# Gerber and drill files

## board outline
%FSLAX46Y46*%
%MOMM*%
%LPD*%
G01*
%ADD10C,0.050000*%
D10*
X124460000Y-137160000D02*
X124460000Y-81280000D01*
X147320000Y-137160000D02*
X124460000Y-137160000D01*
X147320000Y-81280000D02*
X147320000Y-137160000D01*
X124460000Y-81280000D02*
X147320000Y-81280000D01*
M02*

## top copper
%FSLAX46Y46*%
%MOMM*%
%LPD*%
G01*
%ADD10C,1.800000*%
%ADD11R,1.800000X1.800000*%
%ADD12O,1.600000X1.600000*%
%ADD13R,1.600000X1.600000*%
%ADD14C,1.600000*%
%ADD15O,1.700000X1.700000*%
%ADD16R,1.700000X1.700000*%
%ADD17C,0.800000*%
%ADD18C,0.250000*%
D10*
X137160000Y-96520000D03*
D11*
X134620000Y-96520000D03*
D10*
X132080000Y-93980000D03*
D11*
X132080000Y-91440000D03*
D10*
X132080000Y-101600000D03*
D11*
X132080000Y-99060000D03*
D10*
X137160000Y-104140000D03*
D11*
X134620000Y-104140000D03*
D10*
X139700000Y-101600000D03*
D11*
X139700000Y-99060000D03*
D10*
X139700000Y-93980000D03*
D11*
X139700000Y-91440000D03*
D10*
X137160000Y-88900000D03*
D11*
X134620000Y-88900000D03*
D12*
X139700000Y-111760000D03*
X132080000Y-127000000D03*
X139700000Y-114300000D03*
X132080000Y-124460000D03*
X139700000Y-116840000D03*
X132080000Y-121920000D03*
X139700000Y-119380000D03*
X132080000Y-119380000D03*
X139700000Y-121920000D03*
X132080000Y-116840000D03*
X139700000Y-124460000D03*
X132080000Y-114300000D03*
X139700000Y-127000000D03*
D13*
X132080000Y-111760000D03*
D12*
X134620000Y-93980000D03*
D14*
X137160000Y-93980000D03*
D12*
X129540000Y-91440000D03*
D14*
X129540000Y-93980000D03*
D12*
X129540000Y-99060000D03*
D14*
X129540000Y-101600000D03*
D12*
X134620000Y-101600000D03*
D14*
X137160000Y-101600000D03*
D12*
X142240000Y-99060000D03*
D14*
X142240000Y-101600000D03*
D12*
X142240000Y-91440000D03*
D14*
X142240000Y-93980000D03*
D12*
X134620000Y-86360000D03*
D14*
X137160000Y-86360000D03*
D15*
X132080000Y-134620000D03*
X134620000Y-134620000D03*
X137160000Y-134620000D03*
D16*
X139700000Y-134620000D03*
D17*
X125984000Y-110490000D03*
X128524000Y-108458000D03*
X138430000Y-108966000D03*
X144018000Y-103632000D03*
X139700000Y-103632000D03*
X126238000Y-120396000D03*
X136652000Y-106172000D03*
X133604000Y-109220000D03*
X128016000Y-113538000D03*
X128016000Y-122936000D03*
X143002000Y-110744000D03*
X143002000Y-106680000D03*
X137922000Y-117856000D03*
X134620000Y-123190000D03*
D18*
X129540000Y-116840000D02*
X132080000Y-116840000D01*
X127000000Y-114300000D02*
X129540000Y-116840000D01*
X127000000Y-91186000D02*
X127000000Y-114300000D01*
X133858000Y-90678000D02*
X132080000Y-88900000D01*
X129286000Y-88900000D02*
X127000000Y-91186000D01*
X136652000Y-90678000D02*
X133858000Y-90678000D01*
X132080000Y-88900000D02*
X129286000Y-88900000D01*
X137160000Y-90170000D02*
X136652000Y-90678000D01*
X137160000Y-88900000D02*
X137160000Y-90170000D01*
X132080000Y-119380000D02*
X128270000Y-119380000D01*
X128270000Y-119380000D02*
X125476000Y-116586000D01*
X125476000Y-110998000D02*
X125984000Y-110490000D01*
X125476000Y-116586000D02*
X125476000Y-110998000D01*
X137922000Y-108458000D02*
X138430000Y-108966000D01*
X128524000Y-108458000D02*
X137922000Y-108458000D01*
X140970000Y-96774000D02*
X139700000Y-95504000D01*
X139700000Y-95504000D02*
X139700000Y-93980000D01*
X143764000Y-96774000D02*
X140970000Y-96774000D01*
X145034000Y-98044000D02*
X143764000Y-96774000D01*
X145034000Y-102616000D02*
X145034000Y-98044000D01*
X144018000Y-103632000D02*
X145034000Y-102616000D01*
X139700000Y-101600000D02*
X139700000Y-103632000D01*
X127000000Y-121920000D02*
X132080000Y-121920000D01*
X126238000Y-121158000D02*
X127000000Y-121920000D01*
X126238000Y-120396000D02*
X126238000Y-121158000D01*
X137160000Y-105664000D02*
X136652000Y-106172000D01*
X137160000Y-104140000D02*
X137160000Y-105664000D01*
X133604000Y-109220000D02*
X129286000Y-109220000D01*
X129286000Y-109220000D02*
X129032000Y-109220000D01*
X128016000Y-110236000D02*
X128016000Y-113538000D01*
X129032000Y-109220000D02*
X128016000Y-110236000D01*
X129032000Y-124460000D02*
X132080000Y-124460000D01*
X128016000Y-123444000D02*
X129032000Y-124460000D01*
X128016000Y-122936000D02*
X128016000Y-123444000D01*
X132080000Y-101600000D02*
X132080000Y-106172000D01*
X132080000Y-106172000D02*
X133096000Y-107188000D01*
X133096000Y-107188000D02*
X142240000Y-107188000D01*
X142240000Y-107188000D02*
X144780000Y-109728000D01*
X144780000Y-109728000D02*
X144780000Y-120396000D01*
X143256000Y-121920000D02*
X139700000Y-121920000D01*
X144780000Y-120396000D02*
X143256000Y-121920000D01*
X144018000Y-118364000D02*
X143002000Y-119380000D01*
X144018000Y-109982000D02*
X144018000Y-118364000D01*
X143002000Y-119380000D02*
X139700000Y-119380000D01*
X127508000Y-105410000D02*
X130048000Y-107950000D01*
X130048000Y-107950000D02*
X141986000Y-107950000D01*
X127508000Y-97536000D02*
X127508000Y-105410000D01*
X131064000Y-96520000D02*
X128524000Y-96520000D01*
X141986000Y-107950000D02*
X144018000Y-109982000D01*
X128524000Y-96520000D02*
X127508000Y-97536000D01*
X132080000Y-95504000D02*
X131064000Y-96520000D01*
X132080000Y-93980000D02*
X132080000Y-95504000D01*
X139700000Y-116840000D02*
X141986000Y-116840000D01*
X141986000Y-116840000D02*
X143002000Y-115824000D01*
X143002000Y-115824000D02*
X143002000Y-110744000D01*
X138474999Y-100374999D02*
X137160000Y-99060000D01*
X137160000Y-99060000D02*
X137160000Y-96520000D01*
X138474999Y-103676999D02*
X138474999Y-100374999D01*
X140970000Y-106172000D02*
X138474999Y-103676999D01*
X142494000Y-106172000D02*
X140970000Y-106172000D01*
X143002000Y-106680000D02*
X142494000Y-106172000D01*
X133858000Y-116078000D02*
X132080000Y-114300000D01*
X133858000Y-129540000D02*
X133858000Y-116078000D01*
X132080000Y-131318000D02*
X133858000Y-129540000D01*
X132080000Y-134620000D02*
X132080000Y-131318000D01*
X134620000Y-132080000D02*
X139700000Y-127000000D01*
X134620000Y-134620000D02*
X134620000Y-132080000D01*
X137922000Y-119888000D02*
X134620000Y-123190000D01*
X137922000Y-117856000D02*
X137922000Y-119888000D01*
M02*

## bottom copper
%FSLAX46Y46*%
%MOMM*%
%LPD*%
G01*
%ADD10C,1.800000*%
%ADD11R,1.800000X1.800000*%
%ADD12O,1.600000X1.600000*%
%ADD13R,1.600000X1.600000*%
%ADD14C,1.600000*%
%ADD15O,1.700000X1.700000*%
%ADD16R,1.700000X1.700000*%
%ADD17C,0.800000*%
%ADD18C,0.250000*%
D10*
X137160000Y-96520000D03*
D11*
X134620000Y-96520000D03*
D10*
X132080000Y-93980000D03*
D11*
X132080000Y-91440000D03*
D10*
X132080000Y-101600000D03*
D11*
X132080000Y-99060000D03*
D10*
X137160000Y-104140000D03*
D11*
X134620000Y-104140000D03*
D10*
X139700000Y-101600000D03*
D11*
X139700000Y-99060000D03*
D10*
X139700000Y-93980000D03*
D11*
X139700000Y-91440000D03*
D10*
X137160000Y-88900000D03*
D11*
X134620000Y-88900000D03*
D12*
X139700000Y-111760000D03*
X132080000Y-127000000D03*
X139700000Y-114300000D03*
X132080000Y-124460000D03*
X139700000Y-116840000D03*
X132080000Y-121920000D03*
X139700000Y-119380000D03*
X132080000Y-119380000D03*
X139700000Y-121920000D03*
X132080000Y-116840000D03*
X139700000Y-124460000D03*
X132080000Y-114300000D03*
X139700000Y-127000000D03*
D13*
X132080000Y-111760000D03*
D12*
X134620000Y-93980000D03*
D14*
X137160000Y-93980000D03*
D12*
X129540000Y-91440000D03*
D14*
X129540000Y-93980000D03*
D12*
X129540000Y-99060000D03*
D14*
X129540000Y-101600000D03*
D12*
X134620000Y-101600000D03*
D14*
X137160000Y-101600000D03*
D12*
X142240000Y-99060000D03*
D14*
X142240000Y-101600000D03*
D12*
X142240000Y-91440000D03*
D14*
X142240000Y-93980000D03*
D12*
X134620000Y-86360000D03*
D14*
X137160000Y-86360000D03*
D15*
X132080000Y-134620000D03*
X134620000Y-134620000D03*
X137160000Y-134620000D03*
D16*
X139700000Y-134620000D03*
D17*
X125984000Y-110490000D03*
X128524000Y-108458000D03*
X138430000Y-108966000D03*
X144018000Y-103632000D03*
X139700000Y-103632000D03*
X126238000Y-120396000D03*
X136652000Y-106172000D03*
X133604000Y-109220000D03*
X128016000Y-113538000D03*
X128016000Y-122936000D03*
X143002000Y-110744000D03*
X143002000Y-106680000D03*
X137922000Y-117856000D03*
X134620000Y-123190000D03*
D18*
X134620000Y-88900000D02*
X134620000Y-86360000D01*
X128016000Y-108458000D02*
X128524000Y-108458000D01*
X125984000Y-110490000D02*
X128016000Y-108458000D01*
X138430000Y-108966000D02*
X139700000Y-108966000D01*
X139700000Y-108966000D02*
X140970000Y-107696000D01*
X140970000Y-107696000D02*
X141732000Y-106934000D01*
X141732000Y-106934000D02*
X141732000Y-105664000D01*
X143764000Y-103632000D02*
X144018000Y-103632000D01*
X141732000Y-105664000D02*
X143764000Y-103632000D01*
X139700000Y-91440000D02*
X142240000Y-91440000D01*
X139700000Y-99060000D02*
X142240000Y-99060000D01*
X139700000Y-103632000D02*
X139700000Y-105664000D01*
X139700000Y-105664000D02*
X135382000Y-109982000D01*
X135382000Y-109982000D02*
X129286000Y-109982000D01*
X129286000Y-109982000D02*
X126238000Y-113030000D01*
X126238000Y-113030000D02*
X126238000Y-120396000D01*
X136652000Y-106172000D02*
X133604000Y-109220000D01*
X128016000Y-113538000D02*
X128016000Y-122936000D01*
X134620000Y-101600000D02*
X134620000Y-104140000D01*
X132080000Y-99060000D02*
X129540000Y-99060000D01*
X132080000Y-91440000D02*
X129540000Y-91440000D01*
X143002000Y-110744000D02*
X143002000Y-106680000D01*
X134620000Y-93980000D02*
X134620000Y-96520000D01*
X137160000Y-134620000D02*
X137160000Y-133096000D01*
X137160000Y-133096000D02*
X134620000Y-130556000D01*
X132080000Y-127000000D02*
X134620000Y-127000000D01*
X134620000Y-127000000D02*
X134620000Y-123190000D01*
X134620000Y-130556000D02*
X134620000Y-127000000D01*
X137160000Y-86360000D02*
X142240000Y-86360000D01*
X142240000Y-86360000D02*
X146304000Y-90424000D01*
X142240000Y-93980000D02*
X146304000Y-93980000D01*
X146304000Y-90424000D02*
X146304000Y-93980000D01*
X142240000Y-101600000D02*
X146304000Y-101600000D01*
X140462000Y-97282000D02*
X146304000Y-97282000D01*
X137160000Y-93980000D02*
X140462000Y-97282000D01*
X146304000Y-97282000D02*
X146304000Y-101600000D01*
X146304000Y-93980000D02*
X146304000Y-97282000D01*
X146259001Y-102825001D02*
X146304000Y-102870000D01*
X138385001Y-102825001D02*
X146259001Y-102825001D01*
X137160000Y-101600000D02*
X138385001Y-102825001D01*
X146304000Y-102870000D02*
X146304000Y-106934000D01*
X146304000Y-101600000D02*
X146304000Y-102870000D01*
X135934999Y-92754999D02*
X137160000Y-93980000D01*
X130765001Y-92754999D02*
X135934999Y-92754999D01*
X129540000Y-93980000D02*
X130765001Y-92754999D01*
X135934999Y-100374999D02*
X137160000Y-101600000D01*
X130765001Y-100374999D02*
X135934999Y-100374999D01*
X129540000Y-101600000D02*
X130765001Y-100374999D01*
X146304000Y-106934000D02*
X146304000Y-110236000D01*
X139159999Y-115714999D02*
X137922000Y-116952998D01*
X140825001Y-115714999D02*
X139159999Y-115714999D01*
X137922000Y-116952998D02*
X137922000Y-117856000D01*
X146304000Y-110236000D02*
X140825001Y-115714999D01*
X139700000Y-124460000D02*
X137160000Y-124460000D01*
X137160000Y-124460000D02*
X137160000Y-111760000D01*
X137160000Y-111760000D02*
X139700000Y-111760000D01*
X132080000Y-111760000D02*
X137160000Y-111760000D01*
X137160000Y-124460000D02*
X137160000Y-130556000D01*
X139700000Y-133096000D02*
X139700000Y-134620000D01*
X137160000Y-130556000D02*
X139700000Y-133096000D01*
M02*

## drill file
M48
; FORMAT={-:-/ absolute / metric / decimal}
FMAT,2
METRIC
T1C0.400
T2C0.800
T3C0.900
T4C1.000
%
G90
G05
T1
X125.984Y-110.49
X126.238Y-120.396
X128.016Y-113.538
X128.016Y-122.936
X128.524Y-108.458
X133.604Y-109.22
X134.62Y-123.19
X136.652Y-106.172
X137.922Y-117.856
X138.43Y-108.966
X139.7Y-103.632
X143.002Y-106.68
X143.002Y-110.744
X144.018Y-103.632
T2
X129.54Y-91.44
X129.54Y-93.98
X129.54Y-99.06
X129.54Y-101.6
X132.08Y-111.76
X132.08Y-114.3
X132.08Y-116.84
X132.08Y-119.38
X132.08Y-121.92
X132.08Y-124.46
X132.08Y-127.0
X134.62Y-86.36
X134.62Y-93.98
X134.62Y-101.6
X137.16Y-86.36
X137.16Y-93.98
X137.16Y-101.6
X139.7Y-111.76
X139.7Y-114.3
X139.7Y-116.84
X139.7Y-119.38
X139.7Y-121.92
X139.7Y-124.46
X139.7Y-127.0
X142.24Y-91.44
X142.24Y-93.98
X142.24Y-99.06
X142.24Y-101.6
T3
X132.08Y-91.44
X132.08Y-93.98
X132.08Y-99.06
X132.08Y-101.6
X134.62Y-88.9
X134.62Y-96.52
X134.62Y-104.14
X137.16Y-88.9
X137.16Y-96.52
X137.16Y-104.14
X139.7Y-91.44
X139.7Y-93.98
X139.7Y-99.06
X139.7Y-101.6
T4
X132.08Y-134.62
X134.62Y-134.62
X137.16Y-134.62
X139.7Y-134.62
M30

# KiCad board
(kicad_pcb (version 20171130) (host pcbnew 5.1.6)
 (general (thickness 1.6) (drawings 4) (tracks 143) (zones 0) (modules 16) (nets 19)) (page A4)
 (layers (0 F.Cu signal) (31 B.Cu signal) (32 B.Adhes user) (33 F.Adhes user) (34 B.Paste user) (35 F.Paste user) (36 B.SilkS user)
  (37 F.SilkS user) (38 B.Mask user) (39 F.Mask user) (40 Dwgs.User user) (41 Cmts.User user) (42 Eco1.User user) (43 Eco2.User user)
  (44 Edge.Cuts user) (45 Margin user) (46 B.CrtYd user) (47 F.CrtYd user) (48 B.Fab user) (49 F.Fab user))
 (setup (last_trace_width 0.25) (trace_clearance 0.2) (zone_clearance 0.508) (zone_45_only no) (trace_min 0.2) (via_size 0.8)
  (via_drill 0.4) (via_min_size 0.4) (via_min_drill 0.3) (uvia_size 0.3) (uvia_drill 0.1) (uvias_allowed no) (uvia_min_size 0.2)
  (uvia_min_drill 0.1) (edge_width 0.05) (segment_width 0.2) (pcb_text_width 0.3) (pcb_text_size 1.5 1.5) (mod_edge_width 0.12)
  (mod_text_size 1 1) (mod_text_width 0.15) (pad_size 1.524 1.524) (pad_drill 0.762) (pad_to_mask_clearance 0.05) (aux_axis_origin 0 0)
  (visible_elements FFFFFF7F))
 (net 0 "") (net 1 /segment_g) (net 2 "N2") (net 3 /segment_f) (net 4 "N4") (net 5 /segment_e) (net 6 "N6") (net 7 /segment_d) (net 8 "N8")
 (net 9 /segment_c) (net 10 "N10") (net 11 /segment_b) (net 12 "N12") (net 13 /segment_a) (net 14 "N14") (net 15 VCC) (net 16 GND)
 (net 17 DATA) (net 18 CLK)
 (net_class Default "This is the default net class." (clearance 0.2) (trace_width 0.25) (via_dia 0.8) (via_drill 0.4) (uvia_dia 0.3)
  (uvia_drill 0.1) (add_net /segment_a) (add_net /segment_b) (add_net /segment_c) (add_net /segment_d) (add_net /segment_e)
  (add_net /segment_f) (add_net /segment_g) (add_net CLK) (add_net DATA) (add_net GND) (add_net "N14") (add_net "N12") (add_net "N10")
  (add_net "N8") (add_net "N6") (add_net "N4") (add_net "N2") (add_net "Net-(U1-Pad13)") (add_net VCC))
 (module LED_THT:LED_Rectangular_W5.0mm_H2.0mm (layer F.Cu) (at 134.62 96.52)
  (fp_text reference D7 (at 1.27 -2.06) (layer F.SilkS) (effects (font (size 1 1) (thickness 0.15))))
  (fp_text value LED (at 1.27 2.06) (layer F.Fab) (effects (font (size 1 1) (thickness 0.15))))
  (pad 2 thru_hole circle (at 2.54 0) (size 1.8 1.8) (drill 0.9) (layers *.Cu *.Mask) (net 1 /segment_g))
  (pad 1 thru_hole rect (at 0 0) (size 1.8 1.8) (drill 0.9) (layers *.Cu *.Mask) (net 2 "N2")))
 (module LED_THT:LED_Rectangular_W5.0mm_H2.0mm (layer F.Cu) (at 132.08 91.44 270)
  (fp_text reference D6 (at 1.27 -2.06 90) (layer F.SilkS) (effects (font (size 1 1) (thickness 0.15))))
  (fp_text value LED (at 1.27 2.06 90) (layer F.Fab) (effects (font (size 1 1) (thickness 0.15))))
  (pad 2 thru_hole circle (at 2.54 0 270) (size 1.8 1.8) (drill 0.9) (layers *.Cu *.Mask) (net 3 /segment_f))
  (pad 1 thru_hole rect (at 0 0 270) (size 1.8 1.8) (drill 0.9) (layers *.Cu *.Mask) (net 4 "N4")))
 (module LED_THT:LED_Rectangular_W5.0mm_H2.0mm (layer F.Cu) (at 132.08 99.06 270)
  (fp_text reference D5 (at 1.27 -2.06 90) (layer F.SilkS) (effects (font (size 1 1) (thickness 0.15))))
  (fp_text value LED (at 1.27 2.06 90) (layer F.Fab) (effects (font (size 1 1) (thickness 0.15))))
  (pad 2 thru_hole circle (at 2.54 0 270) (size 1.8 1.8) (drill 0.9) (layers *.Cu *.Mask) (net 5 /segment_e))
  (pad 1 thru_hole rect (at 0 0 270) (size 1.8 1.8) (drill 0.9) (layers *.Cu *.Mask) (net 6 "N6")))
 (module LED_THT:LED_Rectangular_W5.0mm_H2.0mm (layer F.Cu) (at 134.62 104.14)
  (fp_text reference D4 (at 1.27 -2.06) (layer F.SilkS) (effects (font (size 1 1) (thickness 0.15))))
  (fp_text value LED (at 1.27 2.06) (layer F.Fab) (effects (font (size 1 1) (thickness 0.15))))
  (pad 2 thru_hole circle (at 2.54 0) (size 1.8 1.8) (drill 0.9) (layers *.Cu *.Mask) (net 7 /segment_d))
  (pad 1 thru_hole rect (at 0 0) (size 1.8 1.8) (drill 0.9) (layers *.Cu *.Mask) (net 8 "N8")))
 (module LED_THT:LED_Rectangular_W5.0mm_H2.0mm (layer F.Cu) (at 139.7 99.06 270)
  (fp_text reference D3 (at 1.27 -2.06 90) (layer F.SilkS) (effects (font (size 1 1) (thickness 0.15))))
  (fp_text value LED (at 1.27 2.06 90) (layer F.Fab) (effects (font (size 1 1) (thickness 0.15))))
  (pad 2 thru_hole circle (at 2.54 0 270) (size 1.8 1.8) (drill 0.9) (layers *.Cu *.Mask) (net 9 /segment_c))
  (pad 1 thru_hole rect (at 0 0 270) (size 1.8 1.8) (drill 0.9) (layers *.Cu *.Mask) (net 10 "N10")))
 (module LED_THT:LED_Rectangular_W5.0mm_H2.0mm (layer F.Cu) (at 139.7 91.44 270)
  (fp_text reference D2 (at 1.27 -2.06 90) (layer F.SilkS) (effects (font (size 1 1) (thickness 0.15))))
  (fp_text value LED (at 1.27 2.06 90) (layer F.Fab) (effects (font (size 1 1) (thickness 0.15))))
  (pad 2 thru_hole circle (at 2.54 0 270) (size 1.8 1.8) (drill 0.9) (layers *.Cu *.Mask) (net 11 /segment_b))
  (pad 1 thru_hole rect (at 0 0 270) (size 1.8 1.8) (drill 0.9) (layers *.Cu *.Mask) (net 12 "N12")))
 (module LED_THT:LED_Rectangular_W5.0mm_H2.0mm (layer F.Cu) (at 134.62 88.9)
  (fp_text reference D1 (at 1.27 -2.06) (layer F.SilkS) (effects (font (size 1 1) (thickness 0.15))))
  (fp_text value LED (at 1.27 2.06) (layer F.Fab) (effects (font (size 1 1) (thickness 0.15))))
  (pad 2 thru_hole circle (at 2.54 0) (size 1.8 1.8) (drill 0.9) (layers *.Cu *.Mask) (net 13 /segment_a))
  (pad 1 thru_hole rect (at 0 0) (size 1.8 1.8) (drill 0.9) (layers *.Cu *.Mask) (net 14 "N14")))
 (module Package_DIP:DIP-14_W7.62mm (layer F.Cu) (at 132.08 111.76)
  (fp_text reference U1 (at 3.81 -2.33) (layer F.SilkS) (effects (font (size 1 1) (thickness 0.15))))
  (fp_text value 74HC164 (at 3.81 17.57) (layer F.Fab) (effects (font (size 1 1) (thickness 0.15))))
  (pad 14 thru_hole oval (at 7.62 0) (size 1.6 1.6) (drill 0.8) (layers *.Cu *.Mask) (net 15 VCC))
  (pad 7 thru_hole oval (at 0 15.24) (size 1.6 1.6) (drill 0.8) (layers *.Cu *.Mask) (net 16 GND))
  (pad 13 thru_hole oval (at 7.62 2.54) (size 1.6 1.6) (drill 0.8) (layers *.Cu *.Mask))
  (pad 6 thru_hole oval (at 0 12.7) (size 1.6 1.6) (drill 0.8) (layers *.Cu *.Mask) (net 7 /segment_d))
  (pad 12 thru_hole oval (at 7.62 5.08) (size 1.6 1.6) (drill 0.8) (layers *.Cu *.Mask) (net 1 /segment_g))
  (pad 5 thru_hole oval (at 0 10.16) (size 1.6 1.6) (drill 0.8) (layers *.Cu *.Mask) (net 9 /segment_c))
  (pad 11 thru_hole oval (at 7.62 7.62) (size 1.6 1.6) (drill 0.8) (layers *.Cu *.Mask) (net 3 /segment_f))
  (pad 4 thru_hole oval (at 0 7.62) (size 1.6 1.6) (drill 0.8) (layers *.Cu *.Mask) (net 11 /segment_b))
  (pad 10 thru_hole oval (at 7.62 10.16) (size 1.6 1.6) (drill 0.8) (layers *.Cu *.Mask) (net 5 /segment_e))
  (pad 3 thru_hole oval (at 0 5.08) (size 1.6 1.6) (drill 0.8) (layers *.Cu *.Mask) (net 13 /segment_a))
  (pad 9 thru_hole oval (at 7.62 12.7) (size 1.6 1.6) (drill 0.8) (layers *.Cu *.Mask) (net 15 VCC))
  (pad 2 thru_hole oval (at 0 2.54) (size 1.6 1.6) (drill 0.8) (layers *.Cu *.Mask) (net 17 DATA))
  (pad 8 thru_hole oval (at 7.62 15.24) (size 1.6 1.6) (drill 0.8) (layers *.Cu *.Mask) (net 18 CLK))
  (pad 1 thru_hole rect (at 0 0) (size 1.6 1.6) (drill 0.8) (layers *.Cu *.Mask) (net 15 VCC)))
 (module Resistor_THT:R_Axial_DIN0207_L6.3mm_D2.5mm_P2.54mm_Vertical (layer F.Cu) (at 137.16 93.98 180)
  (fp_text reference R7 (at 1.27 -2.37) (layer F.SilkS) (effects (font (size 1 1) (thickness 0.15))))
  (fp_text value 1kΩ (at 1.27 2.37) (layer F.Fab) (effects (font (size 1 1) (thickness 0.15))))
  (pad 2 thru_hole oval (at 2.54 0 180) (size 1.6 1.6) (drill 0.8) (layers *.Cu *.Mask) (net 2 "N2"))
  (pad 1 thru_hole circle (at 0 0 180) (size 1.6 1.6) (drill 0.8) (layers *.Cu *.Mask) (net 16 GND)))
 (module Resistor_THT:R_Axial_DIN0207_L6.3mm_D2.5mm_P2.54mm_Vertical (layer F.Cu) (at 129.54 93.98 90)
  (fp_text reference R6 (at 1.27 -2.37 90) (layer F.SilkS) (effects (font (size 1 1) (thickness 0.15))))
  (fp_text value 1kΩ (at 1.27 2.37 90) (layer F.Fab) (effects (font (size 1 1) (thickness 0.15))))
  (pad 2 thru_hole oval (at 2.54 0 90) (size 1.6 1.6) (drill 0.8) (layers *.Cu *.Mask) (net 4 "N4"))
  (pad 1 thru_hole circle (at 0 0 90) (size 1.6 1.6) (drill 0.8) (layers *.Cu *.Mask) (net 16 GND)))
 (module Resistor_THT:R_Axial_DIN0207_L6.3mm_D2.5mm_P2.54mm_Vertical (layer F.Cu) (at 129.54 101.6 90)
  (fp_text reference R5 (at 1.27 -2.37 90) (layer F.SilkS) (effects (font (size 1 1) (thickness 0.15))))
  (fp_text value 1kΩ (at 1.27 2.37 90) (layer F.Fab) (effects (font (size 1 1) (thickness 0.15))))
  (pad 2 thru_hole oval (at 2.54 0 90) (size 1.6 1.6) (drill 0.8) (layers *.Cu *.Mask) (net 6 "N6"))
  (pad 1 thru_hole circle (at 0 0 90) (size 1.6 1.6) (drill 0.8) (layers *.Cu *.Mask) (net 16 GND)))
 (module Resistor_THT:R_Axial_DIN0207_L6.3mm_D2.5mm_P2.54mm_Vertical (layer F.Cu) (at 137.16 101.6 180)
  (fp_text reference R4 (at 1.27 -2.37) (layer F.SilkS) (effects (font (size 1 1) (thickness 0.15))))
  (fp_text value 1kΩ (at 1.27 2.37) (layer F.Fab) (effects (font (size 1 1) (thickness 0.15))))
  (pad 2 thru_hole oval (at 2.54 0 180) (size 1.6 1.6) (drill 0.8) (layers *.Cu *.Mask) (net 8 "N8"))
  (pad 1 thru_hole circle (at 0 0 180) (size 1.6 1.6) (drill 0.8) (layers *.Cu *.Mask) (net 16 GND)))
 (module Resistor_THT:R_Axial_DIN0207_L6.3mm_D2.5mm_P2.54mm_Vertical (layer F.Cu) (at 142.24 101.6 90)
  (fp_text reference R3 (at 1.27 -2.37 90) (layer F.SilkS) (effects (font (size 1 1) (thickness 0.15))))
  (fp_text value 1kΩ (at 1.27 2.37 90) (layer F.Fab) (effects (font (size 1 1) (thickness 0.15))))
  (pad 2 thru_hole oval (at 2.54 0 90) (size 1.6 1.6) (drill 0.8) (layers *.Cu *.Mask) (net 10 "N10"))
  (pad 1 thru_hole circle (at 0 0 90) (size 1.6 1.6) (drill 0.8) (layers *.Cu *.Mask) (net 16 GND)))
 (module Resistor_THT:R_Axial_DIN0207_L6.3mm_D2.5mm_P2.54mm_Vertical (layer F.Cu) (at 142.24 93.98 90)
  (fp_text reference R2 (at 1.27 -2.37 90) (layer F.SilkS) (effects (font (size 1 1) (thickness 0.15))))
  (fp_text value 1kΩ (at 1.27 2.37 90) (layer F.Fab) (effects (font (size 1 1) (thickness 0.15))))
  (pad 2 thru_hole oval (at 2.54 0 90) (size 1.6 1.6) (drill 0.8) (layers *.Cu *.Mask) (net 12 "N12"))
  (pad 1 thru_hole circle (at 0 0 90) (size 1.6 1.6) (drill 0.8) (layers *.Cu *.Mask) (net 16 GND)))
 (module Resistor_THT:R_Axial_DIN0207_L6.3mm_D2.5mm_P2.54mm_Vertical (layer F.Cu) (at 137.16 86.36 180)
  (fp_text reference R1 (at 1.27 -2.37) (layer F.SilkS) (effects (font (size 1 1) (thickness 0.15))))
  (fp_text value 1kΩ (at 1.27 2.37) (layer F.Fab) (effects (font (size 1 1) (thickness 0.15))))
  (pad 2 thru_hole oval (at 2.54 0 180) (size 1.6 1.6) (drill 0.8) (layers *.Cu *.Mask) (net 14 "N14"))
  (pad 1 thru_hole circle (at 0 0 180) (size 1.6 1.6) (drill 0.8) (layers *.Cu *.Mask) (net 16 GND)))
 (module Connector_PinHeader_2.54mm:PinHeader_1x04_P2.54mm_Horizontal (layer F.Cu) (at 139.7 134.62 270)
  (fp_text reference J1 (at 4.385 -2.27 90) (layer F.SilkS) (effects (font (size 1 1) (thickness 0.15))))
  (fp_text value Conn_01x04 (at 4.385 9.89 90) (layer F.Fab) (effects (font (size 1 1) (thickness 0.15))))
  (pad 4 thru_hole oval (at 0 7.62 270) (size 1.7 1.7) (drill 1) (layers *.Cu *.Mask) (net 17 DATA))
  (pad 3 thru_hole oval (at 0 5.08 270) (size 1.7 1.7) (drill 1) (layers *.Cu *.Mask) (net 18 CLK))
  (pad 2 thru_hole oval (at 0 2.54 270) (size 1.7 1.7) (drill 1) (layers *.Cu *.Mask) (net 16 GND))
  (pad 1 thru_hole rect (at 0 0 270) (size 1.7 1.7) (drill 1) (layers *.Cu *.Mask) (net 15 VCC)))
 (gr_line (start 124.46 137.16) (end 124.46 81.28) (layer Edge.Cuts) (width 0.05))
 (gr_line (start 147.32 137.16) (end 124.46 137.16) (layer Edge.Cuts) (width 0.05))
 (gr_line (start 147.32 81.28) (end 147.32 137.16) (layer Edge.Cuts) (width 0.05))
 (gr_line (start 124.46 81.28) (end 147.32 81.28) (layer Edge.Cuts) (width 0.05))
 (segment (start 129.54 116.84) (end 132.08 116.84) (width 0.25) (layer F.Cu) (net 13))
 (segment (start 127 114.3) (end 129.54 116.84) (width 0.25) (layer F.Cu) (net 13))
 (segment (start 127 91.186) (end 127 114.3) (width 0.25) (layer F.Cu) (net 13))
 (segment (start 133.858 90.678) (end 132.08 88.9) (width 0.25) (layer F.Cu) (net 13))
 (segment (start 129.286 88.9) (end 127 91.186) (width 0.25) (layer F.Cu) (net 13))
 (segment (start 136.652 90.678) (end 133.858 90.678) (width 0.25) (layer F.Cu) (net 13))
 (segment (start 132.08 88.9) (end 129.286 88.9) (width 0.25) (layer F.Cu) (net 13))
 (segment (start 137.16 90.17) (end 136.652 90.678) (width 0.25) (layer F.Cu) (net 13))
 (segment (start 137.16 88.9) (end 137.16 90.17) (width 0.25) (layer F.Cu) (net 13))
 (segment (start 134.62 88.9) (end 134.62 86.36) (width 0.25) (layer B.Cu) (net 14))
 (segment (start 132.08 119.38) (end 128.27 119.38) (width 0.25) (layer F.Cu) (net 11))
 (segment (start 128.27 119.38) (end 125.476 116.586) (width 0.25) (layer F.Cu) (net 11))
 (via (at 125.984 110.49) (size 0.8) (drill 0.4) (layers F.Cu B.Cu) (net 11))
 (segment (start 125.476 110.998) (end 125.984 110.49) (width 0.25) (layer F.Cu) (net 11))
 (segment (start 125.476 116.586) (end 125.476 110.998) (width 0.25) (layer F.Cu) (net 11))
 (via (at 128.524 108.458) (size 0.8) (drill 0.4) (layers F.Cu B.Cu) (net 11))
 (segment (start 128.016 108.458) (end 128.524 108.458) (width 0.25) (layer B.Cu) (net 11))
 (segment (start 125.984 110.49) (end 128.016 108.458) (width 0.25) (layer B.Cu) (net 11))
 (via (at 138.43 108.966) (size 0.8) (drill 0.4) (layers F.Cu B.Cu) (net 11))
 (segment (start 137.922 108.458) (end 138.43 108.966) (width 0.25) (layer F.Cu) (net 11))
 (segment (start 128.524 108.458) (end 137.922 108.458) (width 0.25) (layer F.Cu) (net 11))
 (segment (start 138.43 108.966) (end 139.7 108.966) (width 0.25) (layer B.Cu) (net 11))
 (segment (start 139.7 108.966) (end 140.97 107.696) (width 0.25) (layer B.Cu) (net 11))
 (segment (start 140.97 107.696) (end 141.732 106.934) (width 0.25) (layer B.Cu) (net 11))
 (segment (start 141.732 106.934) (end 141.732 105.664) (width 0.25) (layer B.Cu) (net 11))
 (via (at 144.018 103.632) (size 0.8) (drill 0.4) (layers F.Cu B.Cu) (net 11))
 (segment (start 143.764 103.632) (end 144.018 103.632) (width 0.25) (layer B.Cu) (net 11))
 (segment (start 141.732 105.664) (end 143.764 103.632) (width 0.25) (layer B.Cu) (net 11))
 (segment (start 140.97 96.774) (end 139.7 95.504) (width 0.25) (layer F.Cu) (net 11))
 (segment (start 139.7 95.504) (end 139.7 93.98) (width 0.25) (layer F.Cu) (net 11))
 (segment (start 143.764 96.774) (end 140.97 96.774) (width 0.25) (layer F.Cu) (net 11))
 (segment (start 145.034 98.044) (end 143.764 96.774) (width 0.25) (layer F.Cu) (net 11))
 (segment (start 145.034 102.616) (end 145.034 98.044) (width 0.25) (layer F.Cu) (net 11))
 (segment (start 144.018 103.632) (end 145.034 102.616) (width 0.25) (layer F.Cu) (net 11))
 (segment (start 139.7 91.44) (end 142.24 91.44) (width 0.25) (layer B.Cu) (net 12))
 (segment (start 139.7 99.06) (end 142.24 99.06) (width 0.25) (layer B.Cu) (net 10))
 (via (at 139.7 103.632) (size 0.8) (drill 0.4) (layers F.Cu B.Cu) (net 9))
 (segment (start 139.7 101.6) (end 139.7 103.632) (width 0.25) (layer F.Cu) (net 9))
 (segment (start 139.7 103.632) (end 139.7 105.664) (width 0.25) (layer B.Cu) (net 9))
 (segment (start 139.7 105.664) (end 135.382 109.982) (width 0.25) (layer B.Cu) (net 9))
 (segment (start 135.382 109.982) (end 129.286 109.982) (width 0.25) (layer B.Cu) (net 9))
 (segment (start 129.286 109.982) (end 126.238 113.03) (width 0.25) (layer B.Cu) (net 9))
 (via (at 126.238 120.396) (size 0.8) (drill 0.4) (layers F.Cu B.Cu) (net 9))
 (segment (start 126.238 113.03) (end 126.238 120.396) (width 0.25) (layer B.Cu) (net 9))
 (segment (start 127 121.92) (end 132.08 121.92) (width 0.25) (layer F.Cu) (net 9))
 (segment (start 126.238 121.158) (end 127 121.92) (width 0.25) (layer F.Cu) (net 9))
 (segment (start 126.238 120.396) (end 126.238 121.158) (width 0.25) (layer F.Cu) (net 9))
 (via (at 136.652 106.172) (size 0.8) (drill 0.4) (layers F.Cu B.Cu) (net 7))
 (segment (start 137.16 105.664) (end 136.652 106.172) (width 0.25) (layer F.Cu) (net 7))
 (segment (start 137.16 104.14) (end 137.16 105.664) (width 0.25) (layer F.Cu) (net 7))
 (via (at 133.604 109.22) (size 0.8) (drill 0.4) (layers F.Cu B.Cu) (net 7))
 (segment (start 136.652 106.172) (end 133.604 109.22) (width 0.25) (layer B.Cu) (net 7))
 (segment (start 133.604 109.22) (end 129.286 109.22) (width 0.25) (layer F.Cu) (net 7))
 (segment (start 129.286 109.22) (end 129.032 109.22) (width 0.25) (layer F.Cu) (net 7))
 (via (at 128.016 113.538) (size 0.8) (drill 0.4) (layers F.Cu B.Cu) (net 7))
 (segment (start 128.016 110.236) (end 128.016 113.538) (width 0.25) (layer F.Cu) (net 7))
 (segment (start 129.032 109.22) (end 128.016 110.236) (width 0.25) (layer F.Cu) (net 7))
 (via (at 128.016 122.936) (size 0.8) (drill 0.4) (layers F.Cu B.Cu) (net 7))
 (segment (start 128.016 113.538) (end 128.016 122.936) (width 0.25) (layer B.Cu) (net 7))
 (segment (start 129.032 124.46) (end 132.08 124.46) (width 0.25) (layer F.Cu) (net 7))
 (segment (start 128.016 123.444) (end 129.032 124.46) (width 0.25) (layer F.Cu) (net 7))
 (segment (start 128.016 122.936) (end 128.016 123.444) (width 0.25) (layer F.Cu) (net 7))
 (segment (start 134.62 101.6) (end 134.62 104.14) (width 0.25) (layer B.Cu) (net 8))
 (segment (start 132.08 101.6) (end 132.08 106.172) (width 0.25) (layer F.Cu) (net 5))
 (segment (start 132.08 106.172) (end 133.096 107.188) (width 0.25) (layer F.Cu) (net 5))
 (segment (start 133.096 107.188) (end 142.24 107.188) (width 0.25) (layer F.Cu) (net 5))
 (segment (start 142.24 107.188) (end 144.78 109.728) (width 0.25) (layer F.Cu) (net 5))
 (segment (start 144.78 109.728) (end 144.78 120.396) (width 0.25) (layer F.Cu) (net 5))
 (segment (start 143.256 121.92) (end 139.7 121.92) (width 0.25) (layer F.Cu) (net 5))
 (segment (start 144.78 120.396) (end 143.256 121.92) (width 0.25) (layer F.Cu) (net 5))
 (segment (start 132.08 99.06) (end 129.54 99.06) (width 0.25) (layer B.Cu) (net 6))
 (segment (start 144.018 118.364) (end 143.002 119.38) (width 0.25) (layer F.Cu) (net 3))
 (segment (start 144.018 109.982) (end 144.018 118.364) (width 0.25) (layer F.Cu) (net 3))
 (segment (start 143.002 119.38) (end 139.7 119.38) (width 0.25) (layer F.Cu) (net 3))
 (segment (start 127.508 105.41) (end 130.048 107.95) (width 0.25) (layer F.Cu) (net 3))
 (segment (start 130.048 107.95) (end 141.986 107.95) (width 0.25) (layer F.Cu) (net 3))
 (segment (start 127.508 97.536) (end 127.508 105.41) (width 0.25) (layer F.Cu) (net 3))
 (segment (start 131.064 96.52) (end 128.524 96.52) (width 0.25) (layer F.Cu) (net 3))
 (segment (start 141.986 107.95) (end 144.018 109.982) (width 0.25) (layer F.Cu) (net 3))
 (segment (start 128.524 96.52) (end 127.508 97.536) (width 0.25) (layer F.Cu) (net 3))
 (segment (start 132.08 95.504) (end 131.064 96.52) (width 0.25) (layer F.Cu) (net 3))
 (segment (start 132.08 93.98) (end 132.08 95.504) (width 0.25) (layer F.Cu) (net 3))
 (segment (start 132.08 91.44) (end 129.54 91.44) (width 0.25) (layer B.Cu) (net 4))
 (segment (start 139.7 116.84) (end 141.986 116.84) (width 0.25) (layer F.Cu) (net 1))
 (segment (start 141.986 116.84) (end 143.002 115.824) (width 0.25) (layer F.Cu) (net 1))
 (via (at 143.002 110.744) (size 0.8) (drill 0.4) (layers F.Cu B.Cu) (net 1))
 (segment (start 143.002 115.824) (end 143.002 110.744) (width 0.25) (layer F.Cu) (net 1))
 (via (at 143.002 106.68) (size 0.8) (drill 0.4) (layers F.Cu B.Cu) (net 1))
 (segment (start 143.002 110.744) (end 143.002 106.68) (width 0.25) (layer B.Cu) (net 1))
 (segment (start 138.474999 100.374999) (end 137.16 99.06) (width 0.25) (layer F.Cu) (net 1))
 (segment (start 137.16 99.06) (end 137.16 96.52) (width 0.25) (layer F.Cu) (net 1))
 (segment (start 138.474999 103.676999) (end 138.474999 100.374999) (width 0.25) (layer F.Cu) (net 1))
 (segment (start 140.97 106.172) (end 138.474999 103.676999) (width 0.25) (layer F.Cu) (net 1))
 (segment (start 142.494 106.172) (end 140.97 106.172) (width 0.25) (layer F.Cu) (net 1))
 (segment (start 143.002 106.68) (end 142.494 106.172) (width 0.25) (layer F.Cu) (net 1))
 (segment (start 134.62 93.98) (end 134.62 96.52) (width 0.25) (layer B.Cu) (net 2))
 (segment (start 133.858 116.078) (end 132.08 114.3) (width 0.25) (layer F.Cu) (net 17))
 (segment (start 133.858 129.54) (end 133.858 116.078) (width 0.25) (layer F.Cu) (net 17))
 (segment (start 132.08 131.318) (end 133.858 129.54) (width 0.25) (layer F.Cu) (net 17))
 (segment (start 132.08 134.62) (end 132.08 131.318) (width 0.25) (layer F.Cu) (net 17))
 (segment (start 134.62 132.08) (end 139.7 127) (width 0.25) (layer F.Cu) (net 18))
 (segment (start 134.62 134.62) (end 134.62 132.08) (width 0.25) (layer F.Cu) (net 18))
 (segment (start 137.16 134.62) (end 137.16 133.096) (width 0.25) (layer B.Cu) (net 16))
 (segment (start 137.16 133.096) (end 134.62 130.556) (width 0.25) (layer B.Cu) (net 16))
 (segment (start 132.08 127) (end 134.62 127) (width 0.25) (layer B.Cu) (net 16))
 (segment (start 134.62 127) (end 134.62 123.19) (width 0.25) (layer B.Cu) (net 16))
 (segment (start 134.62 130.556) (end 134.62 127) (width 0.25) (layer B.Cu) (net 16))
 (segment (start 137.16 86.36) (end 142.24 86.36) (width 0.25) (layer B.Cu) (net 16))
 (segment (start 142.24 86.36) (end 146.304 90.424) (width 0.25) (layer B.Cu) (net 16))
 (segment (start 142.24 93.98) (end 146.304 93.98) (width 0.25) (layer B.Cu) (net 16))
 (segment (start 146.304 90.424) (end 146.304 93.98) (width 0.25) (layer B.Cu) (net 16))
 (segment (start 142.24 101.6) (end 146.304 101.6) (width 0.25) (layer B.Cu) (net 16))
 (segment (start 140.462 97.282) (end 146.304 97.282) (width 0.25) (layer B.Cu) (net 16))
 (segment (start 137.16 93.98) (end 140.462 97.282) (width 0.25) (layer B.Cu) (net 16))
 (segment (start 146.304 97.282) (end 146.304 101.6) (width 0.25) (layer B.Cu) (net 16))
 (segment (start 146.304 93.98) (end 146.304 97.282) (width 0.25) (layer B.Cu) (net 16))
 (segment (start 146.259001 102.825001) (end 146.304 102.87) (width 0.25) (layer B.Cu) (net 16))
 (segment (start 138.385001 102.825001) (end 146.259001 102.825001) (width 0.25) (layer B.Cu) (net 16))
 (segment (start 137.16 101.6) (end 138.385001 102.825001) (width 0.25) (layer B.Cu) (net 16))
 (segment (start 146.304 102.87) (end 146.304 106.934) (width 0.25) (layer B.Cu) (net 16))
 (segment (start 146.304 101.6) (end 146.304 102.87) (width 0.25) (layer B.Cu) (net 16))
 (segment (start 135.934999 92.754999) (end 137.16 93.98) (width 0.25) (layer B.Cu) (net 16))
 (segment (start 130.765001 92.754999) (end 135.934999 92.754999) (width 0.25) (layer B.Cu) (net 16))
 (segment (start 129.54 93.98) (end 130.765001 92.754999) (width 0.25) (layer B.Cu) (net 16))
 (segment (start 135.934999 100.374999) (end 137.16 101.6) (width 0.25) (layer B.Cu) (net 16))
 (segment (start 130.765001 100.374999) (end 135.934999 100.374999) (width 0.25) (layer B.Cu) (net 16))
 (segment (start 129.54 101.6) (end 130.765001 100.374999) (width 0.25) (layer B.Cu) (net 16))
 (segment (start 146.304 106.934) (end 146.304 110.236) (width 0.25) (layer B.Cu) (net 16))
 (via (at 137.922 117.856) (size 0.8) (drill 0.4) (layers F.Cu B.Cu) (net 16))
 (segment (start 139.159999 115.714999) (end 137.922 116.952998) (width 0.25) (layer B.Cu) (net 16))
 (segment (start 140.825001 115.714999) (end 139.159999 115.714999) (width 0.25) (layer B.Cu) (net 16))
 (segment (start 137.922 116.952998) (end 137.922 117.856) (width 0.25) (layer B.Cu) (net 16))
 (segment (start 146.304 110.236) (end 140.825001 115.714999) (width 0.25) (layer B.Cu) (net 16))
 (via (at 134.62 123.19) (size 0.8) (drill 0.4) (layers F.Cu B.Cu) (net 16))
 (segment (start 137.922 119.888) (end 134.62 123.19) (width 0.25) (layer F.Cu) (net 16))
 (segment (start 137.922 117.856) (end 137.922 119.888) (width 0.25) (layer F.Cu) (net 16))
 (segment (start 139.7 124.46) (end 137.16 124.46) (width 0.25) (layer B.Cu) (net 15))
 (segment (start 137.16 124.46) (end 137.16 111.76) (width 0.25) (layer B.Cu) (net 15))
 (segment (start 137.16 111.76) (end 139.7 111.76) (width 0.25) (layer B.Cu) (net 15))
 (segment (start 132.08 111.76) (end 137.16 111.76) (width 0.25) (layer B.Cu) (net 15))
 (segment (start 137.16 124.46) (end 137.16 130.556) (width 0.25) (layer B.Cu) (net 15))
 (segment (start 139.7 133.096) (end 139.7 134.62) (width 0.25) (layer B.Cu) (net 15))
 (segment (start 137.16 130.556) (end 139.7 133.096) (width 0.25) (layer B.Cu) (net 15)))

